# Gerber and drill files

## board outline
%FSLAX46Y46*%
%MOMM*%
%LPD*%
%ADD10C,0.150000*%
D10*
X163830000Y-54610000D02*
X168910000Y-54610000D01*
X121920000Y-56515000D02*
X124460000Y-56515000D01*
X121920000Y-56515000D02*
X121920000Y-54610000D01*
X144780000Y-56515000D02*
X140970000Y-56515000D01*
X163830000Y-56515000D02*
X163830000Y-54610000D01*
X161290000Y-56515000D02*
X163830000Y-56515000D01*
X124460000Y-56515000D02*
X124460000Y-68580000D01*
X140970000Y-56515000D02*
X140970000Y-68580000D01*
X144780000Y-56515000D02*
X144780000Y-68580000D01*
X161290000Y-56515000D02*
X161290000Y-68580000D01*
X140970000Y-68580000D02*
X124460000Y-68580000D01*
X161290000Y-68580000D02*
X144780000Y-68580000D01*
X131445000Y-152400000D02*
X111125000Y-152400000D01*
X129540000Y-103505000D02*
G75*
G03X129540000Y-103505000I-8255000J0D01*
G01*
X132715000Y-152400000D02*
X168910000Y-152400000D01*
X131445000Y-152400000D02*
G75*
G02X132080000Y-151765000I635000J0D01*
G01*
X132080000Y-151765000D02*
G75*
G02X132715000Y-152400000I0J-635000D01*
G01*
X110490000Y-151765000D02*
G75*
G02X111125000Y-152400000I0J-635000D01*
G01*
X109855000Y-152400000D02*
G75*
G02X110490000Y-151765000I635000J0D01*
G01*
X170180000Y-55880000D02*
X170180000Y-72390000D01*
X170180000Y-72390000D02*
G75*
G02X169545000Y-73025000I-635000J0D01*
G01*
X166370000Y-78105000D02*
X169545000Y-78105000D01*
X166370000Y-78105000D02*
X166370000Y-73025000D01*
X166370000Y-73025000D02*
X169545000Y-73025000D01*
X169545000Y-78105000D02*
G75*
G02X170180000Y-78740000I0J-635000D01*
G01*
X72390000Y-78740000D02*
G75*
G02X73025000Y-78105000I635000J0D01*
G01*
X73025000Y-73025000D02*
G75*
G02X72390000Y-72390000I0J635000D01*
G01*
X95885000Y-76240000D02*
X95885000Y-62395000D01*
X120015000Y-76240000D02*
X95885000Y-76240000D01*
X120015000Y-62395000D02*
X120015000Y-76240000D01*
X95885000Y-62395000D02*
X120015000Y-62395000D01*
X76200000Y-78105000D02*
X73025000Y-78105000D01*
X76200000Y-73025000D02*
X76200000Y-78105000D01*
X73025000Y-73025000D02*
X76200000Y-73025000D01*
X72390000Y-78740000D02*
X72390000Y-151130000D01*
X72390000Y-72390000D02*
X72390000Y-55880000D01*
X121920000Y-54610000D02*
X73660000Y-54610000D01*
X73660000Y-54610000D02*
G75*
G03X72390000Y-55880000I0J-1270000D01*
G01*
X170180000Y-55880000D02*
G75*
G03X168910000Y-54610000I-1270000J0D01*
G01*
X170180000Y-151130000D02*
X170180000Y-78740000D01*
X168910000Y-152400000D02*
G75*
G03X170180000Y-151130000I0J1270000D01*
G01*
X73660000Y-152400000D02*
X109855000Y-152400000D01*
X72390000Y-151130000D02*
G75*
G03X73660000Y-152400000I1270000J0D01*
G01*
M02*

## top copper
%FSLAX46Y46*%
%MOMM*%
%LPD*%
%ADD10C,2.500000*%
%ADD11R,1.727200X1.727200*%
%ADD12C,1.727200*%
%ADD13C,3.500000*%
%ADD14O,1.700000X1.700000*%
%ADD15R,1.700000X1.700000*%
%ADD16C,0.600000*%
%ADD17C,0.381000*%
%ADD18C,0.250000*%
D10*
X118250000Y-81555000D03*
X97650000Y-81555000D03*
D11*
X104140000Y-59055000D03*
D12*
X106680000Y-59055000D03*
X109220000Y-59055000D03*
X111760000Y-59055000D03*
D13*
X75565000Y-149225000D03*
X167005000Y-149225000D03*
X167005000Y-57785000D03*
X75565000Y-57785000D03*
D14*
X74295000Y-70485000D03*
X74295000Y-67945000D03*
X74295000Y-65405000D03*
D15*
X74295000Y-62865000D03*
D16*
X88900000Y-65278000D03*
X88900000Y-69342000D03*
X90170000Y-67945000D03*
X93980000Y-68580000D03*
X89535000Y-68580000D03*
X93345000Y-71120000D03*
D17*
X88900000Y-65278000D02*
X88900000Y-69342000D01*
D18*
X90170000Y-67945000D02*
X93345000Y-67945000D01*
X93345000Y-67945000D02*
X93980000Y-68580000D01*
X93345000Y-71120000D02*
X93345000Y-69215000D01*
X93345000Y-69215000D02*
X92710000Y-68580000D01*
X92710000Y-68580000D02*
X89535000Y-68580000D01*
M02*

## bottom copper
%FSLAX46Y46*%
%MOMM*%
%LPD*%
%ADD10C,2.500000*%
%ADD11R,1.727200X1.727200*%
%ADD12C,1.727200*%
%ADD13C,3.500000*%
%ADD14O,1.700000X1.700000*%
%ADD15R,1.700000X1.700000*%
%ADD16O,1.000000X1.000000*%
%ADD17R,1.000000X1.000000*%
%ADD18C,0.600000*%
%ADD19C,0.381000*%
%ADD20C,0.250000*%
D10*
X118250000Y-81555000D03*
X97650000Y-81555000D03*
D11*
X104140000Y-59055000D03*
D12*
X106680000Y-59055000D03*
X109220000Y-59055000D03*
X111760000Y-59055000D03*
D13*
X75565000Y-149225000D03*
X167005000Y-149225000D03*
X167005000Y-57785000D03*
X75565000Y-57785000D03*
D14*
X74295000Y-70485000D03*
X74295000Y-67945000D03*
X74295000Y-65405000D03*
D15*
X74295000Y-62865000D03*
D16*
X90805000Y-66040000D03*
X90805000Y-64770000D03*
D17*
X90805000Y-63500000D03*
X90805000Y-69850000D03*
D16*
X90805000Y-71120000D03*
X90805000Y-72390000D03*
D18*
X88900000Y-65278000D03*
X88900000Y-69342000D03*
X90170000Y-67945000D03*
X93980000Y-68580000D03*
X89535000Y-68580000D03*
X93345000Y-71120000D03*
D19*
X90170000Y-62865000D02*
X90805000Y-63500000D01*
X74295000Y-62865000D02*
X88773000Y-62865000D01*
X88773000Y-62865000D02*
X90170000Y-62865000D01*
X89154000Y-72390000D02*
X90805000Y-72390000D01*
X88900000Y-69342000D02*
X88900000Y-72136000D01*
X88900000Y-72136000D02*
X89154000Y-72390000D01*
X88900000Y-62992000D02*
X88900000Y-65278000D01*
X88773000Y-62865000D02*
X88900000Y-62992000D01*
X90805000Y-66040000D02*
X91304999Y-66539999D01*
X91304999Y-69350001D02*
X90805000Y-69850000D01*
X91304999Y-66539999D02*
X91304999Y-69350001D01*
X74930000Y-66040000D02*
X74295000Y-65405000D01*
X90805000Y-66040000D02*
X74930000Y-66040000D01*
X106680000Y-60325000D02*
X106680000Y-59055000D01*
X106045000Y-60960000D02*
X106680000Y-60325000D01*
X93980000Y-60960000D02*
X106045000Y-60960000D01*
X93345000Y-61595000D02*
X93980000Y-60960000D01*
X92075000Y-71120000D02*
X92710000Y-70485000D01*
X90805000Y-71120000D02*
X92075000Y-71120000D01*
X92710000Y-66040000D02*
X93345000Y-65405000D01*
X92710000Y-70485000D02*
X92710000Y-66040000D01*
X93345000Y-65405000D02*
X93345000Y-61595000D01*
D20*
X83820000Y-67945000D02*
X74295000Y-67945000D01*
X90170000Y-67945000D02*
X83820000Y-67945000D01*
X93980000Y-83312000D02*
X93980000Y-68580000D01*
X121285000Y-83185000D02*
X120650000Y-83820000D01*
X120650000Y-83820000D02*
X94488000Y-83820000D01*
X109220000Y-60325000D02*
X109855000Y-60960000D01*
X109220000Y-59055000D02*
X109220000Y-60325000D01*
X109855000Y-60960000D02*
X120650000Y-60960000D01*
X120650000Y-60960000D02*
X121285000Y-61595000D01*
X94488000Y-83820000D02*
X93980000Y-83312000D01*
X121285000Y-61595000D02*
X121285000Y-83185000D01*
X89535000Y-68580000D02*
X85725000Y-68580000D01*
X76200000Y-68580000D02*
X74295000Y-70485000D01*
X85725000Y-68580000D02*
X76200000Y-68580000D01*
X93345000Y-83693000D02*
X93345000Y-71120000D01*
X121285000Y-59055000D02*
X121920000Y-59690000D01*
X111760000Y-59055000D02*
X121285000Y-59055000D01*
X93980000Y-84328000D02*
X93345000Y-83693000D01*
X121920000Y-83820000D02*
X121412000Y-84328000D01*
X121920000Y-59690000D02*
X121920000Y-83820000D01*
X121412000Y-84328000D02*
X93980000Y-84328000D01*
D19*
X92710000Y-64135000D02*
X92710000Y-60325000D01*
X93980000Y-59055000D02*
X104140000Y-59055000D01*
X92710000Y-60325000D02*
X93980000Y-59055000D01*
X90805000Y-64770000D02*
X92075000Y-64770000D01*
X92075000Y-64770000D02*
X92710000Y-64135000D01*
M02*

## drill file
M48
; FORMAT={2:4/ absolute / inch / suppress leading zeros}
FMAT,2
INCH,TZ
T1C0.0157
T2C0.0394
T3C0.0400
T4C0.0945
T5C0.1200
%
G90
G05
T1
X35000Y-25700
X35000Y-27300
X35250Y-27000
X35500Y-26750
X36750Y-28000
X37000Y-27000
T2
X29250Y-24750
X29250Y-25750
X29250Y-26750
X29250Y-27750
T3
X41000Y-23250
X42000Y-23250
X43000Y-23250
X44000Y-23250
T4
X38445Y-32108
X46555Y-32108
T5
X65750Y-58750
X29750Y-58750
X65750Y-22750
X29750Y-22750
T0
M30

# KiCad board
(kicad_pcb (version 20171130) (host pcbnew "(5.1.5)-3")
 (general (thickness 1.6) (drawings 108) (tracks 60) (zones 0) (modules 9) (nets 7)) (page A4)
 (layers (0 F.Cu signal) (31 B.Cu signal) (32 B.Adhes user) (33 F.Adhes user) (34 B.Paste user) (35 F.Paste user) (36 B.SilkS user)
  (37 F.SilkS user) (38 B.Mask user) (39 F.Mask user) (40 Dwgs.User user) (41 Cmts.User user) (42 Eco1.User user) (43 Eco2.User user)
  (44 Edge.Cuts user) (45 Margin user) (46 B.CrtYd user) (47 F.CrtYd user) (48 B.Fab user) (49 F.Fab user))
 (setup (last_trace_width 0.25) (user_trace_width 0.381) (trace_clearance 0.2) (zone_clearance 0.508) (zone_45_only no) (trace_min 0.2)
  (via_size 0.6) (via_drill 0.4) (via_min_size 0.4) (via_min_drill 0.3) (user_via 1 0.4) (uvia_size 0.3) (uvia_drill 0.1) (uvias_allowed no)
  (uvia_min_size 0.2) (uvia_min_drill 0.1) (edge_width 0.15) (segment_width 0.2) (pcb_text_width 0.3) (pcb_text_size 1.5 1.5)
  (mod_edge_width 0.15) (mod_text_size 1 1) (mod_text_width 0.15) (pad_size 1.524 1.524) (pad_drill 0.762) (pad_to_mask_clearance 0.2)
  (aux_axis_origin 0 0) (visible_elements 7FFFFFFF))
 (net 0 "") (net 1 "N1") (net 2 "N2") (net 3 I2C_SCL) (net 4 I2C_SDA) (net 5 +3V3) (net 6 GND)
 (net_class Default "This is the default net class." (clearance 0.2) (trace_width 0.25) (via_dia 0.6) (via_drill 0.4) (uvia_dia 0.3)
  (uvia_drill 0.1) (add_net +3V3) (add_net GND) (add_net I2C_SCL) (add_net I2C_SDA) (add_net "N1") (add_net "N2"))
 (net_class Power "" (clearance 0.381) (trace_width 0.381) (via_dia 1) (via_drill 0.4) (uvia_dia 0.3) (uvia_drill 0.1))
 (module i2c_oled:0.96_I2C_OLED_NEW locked (layer F.Cu) (at 107.95 59.055)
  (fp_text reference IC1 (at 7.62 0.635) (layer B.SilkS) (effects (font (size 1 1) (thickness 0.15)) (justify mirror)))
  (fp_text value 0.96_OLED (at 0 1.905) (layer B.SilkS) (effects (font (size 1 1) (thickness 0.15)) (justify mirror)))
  (pad "" np_thru_hole circle (at 10.3 22.5) (size 2.5 2.5) (drill 2.4) (layers *.Cu *.Mask))
  (pad "" np_thru_hole circle (at -10.3 22.5) (size 2.5 2.5) (drill 2.4) (layers *.Cu *.Mask))
  (pad 1 thru_hole rect (at -3.81 0) (size 1.7272 1.7272) (drill 1.016) (layers *.Cu *.Mask) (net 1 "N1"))
  (pad 2 thru_hole circle (at -1.27 0) (size 1.7272 1.7272) (drill 1.016) (layers *.Cu *.Mask) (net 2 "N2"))
  (pad 3 thru_hole circle (at 1.27 0) (size 1.7272 1.7272) (drill 1.016) (layers *.Cu *.Mask) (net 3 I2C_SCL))
  (pad 4 thru_hole circle (at 3.81 0) (size 1.7272 1.7272) (drill 1.016) (layers *.Cu *.Mask) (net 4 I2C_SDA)))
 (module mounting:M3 (layer F.Cu) (at 75.565 149.225)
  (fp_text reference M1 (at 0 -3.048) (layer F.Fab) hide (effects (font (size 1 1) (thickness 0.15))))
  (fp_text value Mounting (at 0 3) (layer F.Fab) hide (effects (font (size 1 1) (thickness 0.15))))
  (pad "" np_thru_hole circle (at 0 0) (size 3.5 3.5) (drill 3.048) (layers *.Cu *.Mask) (solder_mask_margin 0.8)))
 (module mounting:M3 (layer F.Cu) (at 167.005 149.225)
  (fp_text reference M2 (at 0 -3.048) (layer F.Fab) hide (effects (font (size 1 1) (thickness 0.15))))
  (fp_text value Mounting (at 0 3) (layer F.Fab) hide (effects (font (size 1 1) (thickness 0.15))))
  (pad "" np_thru_hole circle (at 0 0) (size 3.5 3.5) (drill 3.048) (layers *.Cu *.Mask) (solder_mask_margin 0.8)))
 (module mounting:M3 (layer F.Cu) (at 167.005 57.785)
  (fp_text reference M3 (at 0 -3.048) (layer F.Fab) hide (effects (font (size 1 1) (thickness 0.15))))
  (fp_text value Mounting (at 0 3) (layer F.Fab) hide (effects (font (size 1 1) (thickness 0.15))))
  (pad "" np_thru_hole circle (at 0 0) (size 3.5 3.5) (drill 3.048) (layers *.Cu *.Mask) (solder_mask_margin 0.8)))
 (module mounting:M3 (layer F.Cu) (at 75.565 57.785)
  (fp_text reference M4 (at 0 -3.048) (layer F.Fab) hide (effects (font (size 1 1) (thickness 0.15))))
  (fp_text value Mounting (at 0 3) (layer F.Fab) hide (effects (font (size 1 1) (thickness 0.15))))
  (pad "" np_thru_hole circle (at 0 0) (size 3.5 3.5) (drill 3.048) (layers *.Cu *.Mask) (solder_mask_margin 0.8)))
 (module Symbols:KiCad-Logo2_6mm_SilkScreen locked (layer B.Cu) (at 142.875 88.9 180)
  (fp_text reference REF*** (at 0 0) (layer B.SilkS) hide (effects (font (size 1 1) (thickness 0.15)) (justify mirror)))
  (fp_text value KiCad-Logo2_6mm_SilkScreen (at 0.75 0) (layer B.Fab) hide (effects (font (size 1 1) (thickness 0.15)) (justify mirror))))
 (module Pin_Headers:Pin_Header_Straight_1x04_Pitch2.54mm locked (layer B.Cu) (at 74.295 62.865 180)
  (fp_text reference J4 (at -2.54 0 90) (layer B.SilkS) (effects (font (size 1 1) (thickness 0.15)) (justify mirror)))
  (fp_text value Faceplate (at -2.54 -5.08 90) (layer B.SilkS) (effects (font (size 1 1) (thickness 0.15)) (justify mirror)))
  (pad 4 thru_hole oval (at 0 -7.62 180) (size 1.7 1.7) (drill 1) (layers *.Cu *.Mask) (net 4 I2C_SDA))
  (pad 3 thru_hole oval (at 0 -5.08 180) (size 1.7 1.7) (drill 1) (layers *.Cu *.Mask) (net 3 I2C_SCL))
  (pad 2 thru_hole oval (at 0 -2.54 180) (size 1.7 1.7) (drill 1) (layers *.Cu *.Mask) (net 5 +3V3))
  (pad 1 thru_hole rect (at 0 0 180) (size 1.7 1.7) (drill 1) (layers *.Cu *.Mask) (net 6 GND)))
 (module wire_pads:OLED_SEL (layer B.Cu) (at 90.805 63.5 180)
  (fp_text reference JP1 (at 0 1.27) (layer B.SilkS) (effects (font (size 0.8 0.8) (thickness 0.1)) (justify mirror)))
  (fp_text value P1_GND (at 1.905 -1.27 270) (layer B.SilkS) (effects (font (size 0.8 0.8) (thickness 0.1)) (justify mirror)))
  (pad 3 smd oval (at 0 -2.54 180) (size 1 1) (layers B.Cu B.Paste B.Mask) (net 5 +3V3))
  (pad 2 smd oval (at 0 -1.27 180) (size 1 1) (layers B.Cu B.Paste B.Mask) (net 1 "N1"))
  (pad 1 smd rect (at 0 0 180) (size 1 1) (layers B.Cu B.Paste B.Mask) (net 6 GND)))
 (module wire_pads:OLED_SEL (layer B.Cu) (at 90.805 69.85 180)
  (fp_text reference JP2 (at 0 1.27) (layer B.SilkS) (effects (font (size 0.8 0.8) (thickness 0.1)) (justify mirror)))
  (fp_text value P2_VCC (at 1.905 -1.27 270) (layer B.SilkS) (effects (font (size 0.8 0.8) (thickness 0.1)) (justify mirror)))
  (pad 1 smd rect (at 0 0 180) (size 1 1) (layers B.Cu B.Paste B.Mask) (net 5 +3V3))
  (pad 2 smd oval (at 0 -1.27 180) (size 1 1) (layers B.Cu B.Paste B.Mask) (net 2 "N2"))
  (pad 3 smd oval (at 0 -2.54 180) (size 1 1) (layers B.Cu B.Paste B.Mask) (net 6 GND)))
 (gr_line (start 163.83 54.61) (end 168.91 54.61) (layer Edge.Cuts) (width 0.15))
 (gr_line (start 121.92 56.515) (end 124.46 56.515) (layer Edge.Cuts) (width 0.15))
 (gr_line (start 121.92 56.515) (end 121.92 54.61) (layer Edge.Cuts) (width 0.15))
 (gr_line (start 144.78 56.515) (end 140.97 56.515) (layer Edge.Cuts) (width 0.15))
 (gr_line (start 163.83 56.515) (end 163.83 54.61) (layer Edge.Cuts) (width 0.15))
 (gr_line (start 161.29 56.515) (end 163.83 56.515) (layer Edge.Cuts) (width 0.15))
 (gr_line (start 124.46 56.515) (end 124.46 68.58) (layer Edge.Cuts) (width 0.15))
 (gr_line (start 140.97 56.515) (end 140.97 68.58) (layer Edge.Cuts) (width 0.15))
 (gr_line (start 144.78 56.515) (end 144.78 68.58) (layer Edge.Cuts) (width 0.15))
 (gr_line (start 161.29 56.515) (end 161.29 68.58) (layer Edge.Cuts) (width 0.15))
 (gr_line (start 140.97 68.58) (end 124.46 68.58) (layer Edge.Cuts) (width 0.15))
 (gr_line (start 161.29 68.58) (end 144.78 68.58) (layer Edge.Cuts) (width 0.15))
 (gr_line (start 131.445 152.4) (end 111.125 152.4) (layer Edge.Cuts) (width 0.15))
 (gr_circle (center 121.285 103.505) (end 129.54 103.505) (layer Edge.Cuts) (width 0.15))
 (gr_line (start 132.715 152.4) (end 168.91 152.4) (layer Edge.Cuts) (width 0.15))
 (gr_arc (start 132.08 152.4) (end 132.08 151.765) (angle -90) (layer Edge.Cuts) (width 0.15))
 (gr_arc (start 132.08 152.4) (end 132.715 152.4) (angle -90) (layer Edge.Cuts) (width 0.15))
 (gr_arc (start 110.49 152.4) (end 111.125 152.4) (angle -90) (layer Edge.Cuts) (width 0.15))
 (gr_arc (start 110.49 152.4) (end 110.49 151.765) (angle -90) (layer Edge.Cuts) (width 0.15))
 (gr_line (start 170.18 55.88) (end 170.18 72.39) (layer Edge.Cuts) (width 0.15))
 (gr_arc (start 169.545 72.39) (end 169.545 73.025) (angle -90) (layer Edge.Cuts) (width 0.15))
 (gr_line (start 166.37 78.105) (end 169.545 78.105) (layer Edge.Cuts) (width 0.15))
 (gr_line (start 166.37 78.105) (end 166.37 73.025) (layer Edge.Cuts) (width 0.15))
 (gr_line (start 166.37 73.025) (end 169.545 73.025) (layer Edge.Cuts) (width 0.15))
 (gr_arc (start 169.545 78.74) (end 170.18 78.74) (angle -90) (layer Edge.Cuts) (width 0.15))
 (gr_arc (start 73.025 78.74) (end 73.025 78.105) (angle -90) (layer Edge.Cuts) (width 0.15))
 (gr_arc (start 73.025 72.39) (end 72.39 72.39) (angle -90) (layer Edge.Cuts) (width 0.15))
 (gr_line (start 95.885 76.24) (end 95.885 62.395) (layer Edge.Cuts) (width 0.15))
 (gr_line (start 120.015 76.24) (end 95.885 76.24) (layer Edge.Cuts) (width 0.15))
 (gr_line (start 120.015 62.395) (end 120.015 76.24) (layer Edge.Cuts) (width 0.15))
 (gr_line (start 95.885 62.395) (end 120.015 62.395) (layer Edge.Cuts) (width 0.15))
 (gr_line (start 76.2 78.105) (end 73.025 78.105) (layer Edge.Cuts) (width 0.15))
 (gr_line (start 76.2 73.025) (end 76.2 78.105) (layer Edge.Cuts) (width 0.15))
 (gr_line (start 73.025 73.025) (end 76.2 73.025) (layer Edge.Cuts) (width 0.15))
 (gr_line (start 72.39 78.74) (end 72.39 151.13) (layer Edge.Cuts) (width 0.15))
 (gr_line (start 72.39 72.39) (end 72.39 55.88) (layer Edge.Cuts) (width 0.15))
 (gr_line (start 121.92 54.61) (end 73.66 54.61) (angle 90) (layer Edge.Cuts) (width 0.15))
 (gr_arc (start 73.66 55.88) (end 72.39 55.88) (angle 90) (layer Edge.Cuts) (width 0.15))
 (gr_arc (start 168.91 55.88) (end 168.91 54.61) (angle 90) (layer Edge.Cuts) (width 0.15))
 (gr_line (start 170.18 151.13) (end 170.18 78.74) (angle 90) (layer Edge.Cuts) (width 0.15))
 (gr_arc (start 168.91 151.13) (end 170.18 151.13) (angle 90) (layer Edge.Cuts) (width 0.15))
 (gr_line (start 73.66 152.4) (end 109.855 152.4) (angle 90) (layer Edge.Cuts) (width 0.15))
 (gr_arc (start 73.66 151.13) (end 73.66 152.4) (angle 90) (layer Edge.Cuts) (width 0.15))
 (segment (start 90.17 62.865) (end 90.805 63.5) (width 0.381) (layer B.Cu) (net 6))
 (via (at 88.9 65.278) (size 0.6) (drill 0.4) (layers F.Cu B.Cu) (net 6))
 (segment (start 74.295 62.865) (end 88.773 62.865) (width 0.381) (layer B.Cu) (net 6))
 (segment (start 88.773 62.865) (end 90.17 62.865) (width 0.381) (layer B.Cu) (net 6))
 (via (at 88.9 69.342) (size 0.6) (drill 0.4) (layers F.Cu B.Cu) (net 6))
 (segment (start 88.9 65.278) (end 88.9 69.342) (width 0.381) (layer F.Cu) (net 6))
 (segment (start 89.154 72.39) (end 90.805 72.39) (width 0.381) (layer B.Cu) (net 6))
 (segment (start 88.9 69.342) (end 88.9 72.136) (width 0.381) (layer B.Cu) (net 6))
 (segment (start 88.9 72.136) (end 89.154 72.39) (width 0.381) (layer B.Cu) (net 6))
 (segment (start 88.9 62.992) (end 88.9 65.278) (width 0.381) (layer B.Cu) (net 6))
 (segment (start 88.773 62.865) (end 88.9 62.992) (width 0.381) (layer B.Cu) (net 6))
 (segment (start 90.805 66.04) (end 91.304999 66.539999) (width 0.381) (layer B.Cu) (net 5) (status 10))
 (segment (start 91.304999 69.350001) (end 90.805 69.85) (width 0.381) (layer B.Cu) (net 5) (status 30))
 (segment (start 91.304999 66.539999) (end 91.304999 69.350001) (width 0.381) (layer B.Cu) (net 5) (status 20))
 (segment (start 74.93 66.04) (end 74.295 65.405) (width 0.381) (layer B.Cu) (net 5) (status 20))
 (segment (start 90.805 66.04) (end 74.93 66.04) (width 0.381) (layer B.Cu) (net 5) (status 10))
 (segment (start 106.68 60.325) (end 106.68 59.055) (width 0.381) (layer B.Cu) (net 2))
 (segment (start 106.045 60.96) (end 106.68 60.325) (width 0.381) (layer B.Cu) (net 2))
 (segment (start 93.98 60.96) (end 106.045 60.96) (width 0.381) (layer B.Cu) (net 2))
 (segment (start 93.345 61.595) (end 93.98 60.96) (width 0.381) (layer B.Cu) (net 2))
 (segment (start 92.075 71.12) (end 92.71 70.485) (width 0.381) (layer B.Cu) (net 2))
 (segment (start 90.805 71.12) (end 92.075 71.12) (width 0.381) (layer B.Cu) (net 2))
 (segment (start 92.71 66.04) (end 93.345 65.405) (width 0.381) (layer B.Cu) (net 2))
 (segment (start 92.71 70.485) (end 92.71 66.04) (width 0.381) (layer B.Cu) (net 2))
 (segment (start 93.345 65.405) (end 93.345 61.595) (width 0.381) (layer B.Cu) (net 2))
 (via (at 90.17 67.945) (size 0.6) (drill 0.4) (layers F.Cu B.Cu) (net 3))
 (segment (start 90.17 67.945) (end 93.345 67.945) (width 0.25) (layer F.Cu) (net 3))
 (segment (start 83.82 67.945) (end 74.295 67.945) (width 0.25) (layer B.Cu) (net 3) (status 20))
 (segment (start 90.17 67.945) (end 83.82 67.945) (width 0.25) (layer B.Cu) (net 3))
 (via (at 93.98 68.58) (size 0.6) (drill 0.4) (layers F.Cu B.Cu) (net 3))
 (segment (start 93.345 67.945) (end 93.98 68.58) (width 0.25) (layer F.Cu) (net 3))
 (segment (start 93.98 83.312) (end 93.98 68.58) (width 0.25) (layer B.Cu) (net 3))
 (segment (start 121.285 83.185) (end 120.65 83.82) (width 0.25) (layer B.Cu) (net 3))
 (segment (start 120.65 83.82) (end 94.488 83.82) (width 0.25) (layer B.Cu) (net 3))
 (segment (start 109.22 60.325) (end 109.855 60.96) (width 0.25) (layer B.Cu) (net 3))
 (segment (start 109.22 59.055) (end 109.22 60.325) (width 0.25) (layer B.Cu) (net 3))
 (segment (start 109.855 60.96) (end 120.65 60.96) (width 0.25) (layer B.Cu) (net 3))
 (segment (start 120.65 60.96) (end 121.285 61.595) (width 0.25) (layer B.Cu) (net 3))
 (segment (start 94.488 83.82) (end 93.98 83.312) (width 0.25) (layer B.Cu) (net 3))
 (segment (start 121.285 61.595) (end 121.285 83.185) (width 0.25) (layer B.Cu) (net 3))
 (via (at 89.535 68.58) (size 0.6) (drill 0.4) (layers F.Cu B.Cu) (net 4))
 (segment (start 89.535 68.58) (end 85.725 68.58) (width 0.25) (layer B.Cu) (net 4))
 (segment (start 76.2 68.58) (end 74.295 70.485) (width 0.25) (layer B.Cu) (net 4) (status 20))
 (segment (start 85.725 68.58) (end 76.2 68.58) (width 0.25) (layer B.Cu) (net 4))
 (via (at 93.345 71.12) (size 0.6) (drill 0.4) (layers F.Cu B.Cu) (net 4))
 (segment (start 93.345 71.12) (end 93.345 69.215) (width 0.25) (layer F.Cu) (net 4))
 (segment (start 93.345 69.215) (end 92.71 68.58) (width 0.25) (layer F.Cu) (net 4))
 (segment (start 92.71 68.58) (end 89.535 68.58) (width 0.25) (layer F.Cu) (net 4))
 (segment (start 93.345 83.693) (end 93.345 71.12) (width 0.25) (layer B.Cu) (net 4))
 (segment (start 121.285 59.055) (end 121.92 59.69) (width 0.25) (layer B.Cu) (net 4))
 (segment (start 111.76 59.055) (end 121.285 59.055) (width 0.25) (layer B.Cu) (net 4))
 (segment (start 93.98 84.328) (end 93.345 83.693) (width 0.25) (layer B.Cu) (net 4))
 (segment (start 121.92 83.82) (end 121.412 84.328) (width 0.25) (layer B.Cu) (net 4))
 (segment (start 121.92 59.69) (end 121.92 83.82) (width 0.25) (layer B.Cu) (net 4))
 (segment (start 121.412 84.328) (end 93.98 84.328) (width 0.25) (layer B.Cu) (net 4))
 (segment (start 92.71 64.135) (end 92.71 60.325) (width 0.381) (layer B.Cu) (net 1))
 (segment (start 93.98 59.055) (end 104.14 59.055) (width 0.381) (layer B.Cu) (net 1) (status 20))
 (segment (start 92.71 60.325) (end 93.98 59.055) (width 0.381) (layer B.Cu) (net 1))
 (segment (start 90.805 64.77) (end 92.075 64.77) (width 0.381) (layer B.Cu) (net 1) (status 10))
 (segment (start 92.075 64.77) (end 92.71 64.135) (width 0.381) (layer B.Cu) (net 1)))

